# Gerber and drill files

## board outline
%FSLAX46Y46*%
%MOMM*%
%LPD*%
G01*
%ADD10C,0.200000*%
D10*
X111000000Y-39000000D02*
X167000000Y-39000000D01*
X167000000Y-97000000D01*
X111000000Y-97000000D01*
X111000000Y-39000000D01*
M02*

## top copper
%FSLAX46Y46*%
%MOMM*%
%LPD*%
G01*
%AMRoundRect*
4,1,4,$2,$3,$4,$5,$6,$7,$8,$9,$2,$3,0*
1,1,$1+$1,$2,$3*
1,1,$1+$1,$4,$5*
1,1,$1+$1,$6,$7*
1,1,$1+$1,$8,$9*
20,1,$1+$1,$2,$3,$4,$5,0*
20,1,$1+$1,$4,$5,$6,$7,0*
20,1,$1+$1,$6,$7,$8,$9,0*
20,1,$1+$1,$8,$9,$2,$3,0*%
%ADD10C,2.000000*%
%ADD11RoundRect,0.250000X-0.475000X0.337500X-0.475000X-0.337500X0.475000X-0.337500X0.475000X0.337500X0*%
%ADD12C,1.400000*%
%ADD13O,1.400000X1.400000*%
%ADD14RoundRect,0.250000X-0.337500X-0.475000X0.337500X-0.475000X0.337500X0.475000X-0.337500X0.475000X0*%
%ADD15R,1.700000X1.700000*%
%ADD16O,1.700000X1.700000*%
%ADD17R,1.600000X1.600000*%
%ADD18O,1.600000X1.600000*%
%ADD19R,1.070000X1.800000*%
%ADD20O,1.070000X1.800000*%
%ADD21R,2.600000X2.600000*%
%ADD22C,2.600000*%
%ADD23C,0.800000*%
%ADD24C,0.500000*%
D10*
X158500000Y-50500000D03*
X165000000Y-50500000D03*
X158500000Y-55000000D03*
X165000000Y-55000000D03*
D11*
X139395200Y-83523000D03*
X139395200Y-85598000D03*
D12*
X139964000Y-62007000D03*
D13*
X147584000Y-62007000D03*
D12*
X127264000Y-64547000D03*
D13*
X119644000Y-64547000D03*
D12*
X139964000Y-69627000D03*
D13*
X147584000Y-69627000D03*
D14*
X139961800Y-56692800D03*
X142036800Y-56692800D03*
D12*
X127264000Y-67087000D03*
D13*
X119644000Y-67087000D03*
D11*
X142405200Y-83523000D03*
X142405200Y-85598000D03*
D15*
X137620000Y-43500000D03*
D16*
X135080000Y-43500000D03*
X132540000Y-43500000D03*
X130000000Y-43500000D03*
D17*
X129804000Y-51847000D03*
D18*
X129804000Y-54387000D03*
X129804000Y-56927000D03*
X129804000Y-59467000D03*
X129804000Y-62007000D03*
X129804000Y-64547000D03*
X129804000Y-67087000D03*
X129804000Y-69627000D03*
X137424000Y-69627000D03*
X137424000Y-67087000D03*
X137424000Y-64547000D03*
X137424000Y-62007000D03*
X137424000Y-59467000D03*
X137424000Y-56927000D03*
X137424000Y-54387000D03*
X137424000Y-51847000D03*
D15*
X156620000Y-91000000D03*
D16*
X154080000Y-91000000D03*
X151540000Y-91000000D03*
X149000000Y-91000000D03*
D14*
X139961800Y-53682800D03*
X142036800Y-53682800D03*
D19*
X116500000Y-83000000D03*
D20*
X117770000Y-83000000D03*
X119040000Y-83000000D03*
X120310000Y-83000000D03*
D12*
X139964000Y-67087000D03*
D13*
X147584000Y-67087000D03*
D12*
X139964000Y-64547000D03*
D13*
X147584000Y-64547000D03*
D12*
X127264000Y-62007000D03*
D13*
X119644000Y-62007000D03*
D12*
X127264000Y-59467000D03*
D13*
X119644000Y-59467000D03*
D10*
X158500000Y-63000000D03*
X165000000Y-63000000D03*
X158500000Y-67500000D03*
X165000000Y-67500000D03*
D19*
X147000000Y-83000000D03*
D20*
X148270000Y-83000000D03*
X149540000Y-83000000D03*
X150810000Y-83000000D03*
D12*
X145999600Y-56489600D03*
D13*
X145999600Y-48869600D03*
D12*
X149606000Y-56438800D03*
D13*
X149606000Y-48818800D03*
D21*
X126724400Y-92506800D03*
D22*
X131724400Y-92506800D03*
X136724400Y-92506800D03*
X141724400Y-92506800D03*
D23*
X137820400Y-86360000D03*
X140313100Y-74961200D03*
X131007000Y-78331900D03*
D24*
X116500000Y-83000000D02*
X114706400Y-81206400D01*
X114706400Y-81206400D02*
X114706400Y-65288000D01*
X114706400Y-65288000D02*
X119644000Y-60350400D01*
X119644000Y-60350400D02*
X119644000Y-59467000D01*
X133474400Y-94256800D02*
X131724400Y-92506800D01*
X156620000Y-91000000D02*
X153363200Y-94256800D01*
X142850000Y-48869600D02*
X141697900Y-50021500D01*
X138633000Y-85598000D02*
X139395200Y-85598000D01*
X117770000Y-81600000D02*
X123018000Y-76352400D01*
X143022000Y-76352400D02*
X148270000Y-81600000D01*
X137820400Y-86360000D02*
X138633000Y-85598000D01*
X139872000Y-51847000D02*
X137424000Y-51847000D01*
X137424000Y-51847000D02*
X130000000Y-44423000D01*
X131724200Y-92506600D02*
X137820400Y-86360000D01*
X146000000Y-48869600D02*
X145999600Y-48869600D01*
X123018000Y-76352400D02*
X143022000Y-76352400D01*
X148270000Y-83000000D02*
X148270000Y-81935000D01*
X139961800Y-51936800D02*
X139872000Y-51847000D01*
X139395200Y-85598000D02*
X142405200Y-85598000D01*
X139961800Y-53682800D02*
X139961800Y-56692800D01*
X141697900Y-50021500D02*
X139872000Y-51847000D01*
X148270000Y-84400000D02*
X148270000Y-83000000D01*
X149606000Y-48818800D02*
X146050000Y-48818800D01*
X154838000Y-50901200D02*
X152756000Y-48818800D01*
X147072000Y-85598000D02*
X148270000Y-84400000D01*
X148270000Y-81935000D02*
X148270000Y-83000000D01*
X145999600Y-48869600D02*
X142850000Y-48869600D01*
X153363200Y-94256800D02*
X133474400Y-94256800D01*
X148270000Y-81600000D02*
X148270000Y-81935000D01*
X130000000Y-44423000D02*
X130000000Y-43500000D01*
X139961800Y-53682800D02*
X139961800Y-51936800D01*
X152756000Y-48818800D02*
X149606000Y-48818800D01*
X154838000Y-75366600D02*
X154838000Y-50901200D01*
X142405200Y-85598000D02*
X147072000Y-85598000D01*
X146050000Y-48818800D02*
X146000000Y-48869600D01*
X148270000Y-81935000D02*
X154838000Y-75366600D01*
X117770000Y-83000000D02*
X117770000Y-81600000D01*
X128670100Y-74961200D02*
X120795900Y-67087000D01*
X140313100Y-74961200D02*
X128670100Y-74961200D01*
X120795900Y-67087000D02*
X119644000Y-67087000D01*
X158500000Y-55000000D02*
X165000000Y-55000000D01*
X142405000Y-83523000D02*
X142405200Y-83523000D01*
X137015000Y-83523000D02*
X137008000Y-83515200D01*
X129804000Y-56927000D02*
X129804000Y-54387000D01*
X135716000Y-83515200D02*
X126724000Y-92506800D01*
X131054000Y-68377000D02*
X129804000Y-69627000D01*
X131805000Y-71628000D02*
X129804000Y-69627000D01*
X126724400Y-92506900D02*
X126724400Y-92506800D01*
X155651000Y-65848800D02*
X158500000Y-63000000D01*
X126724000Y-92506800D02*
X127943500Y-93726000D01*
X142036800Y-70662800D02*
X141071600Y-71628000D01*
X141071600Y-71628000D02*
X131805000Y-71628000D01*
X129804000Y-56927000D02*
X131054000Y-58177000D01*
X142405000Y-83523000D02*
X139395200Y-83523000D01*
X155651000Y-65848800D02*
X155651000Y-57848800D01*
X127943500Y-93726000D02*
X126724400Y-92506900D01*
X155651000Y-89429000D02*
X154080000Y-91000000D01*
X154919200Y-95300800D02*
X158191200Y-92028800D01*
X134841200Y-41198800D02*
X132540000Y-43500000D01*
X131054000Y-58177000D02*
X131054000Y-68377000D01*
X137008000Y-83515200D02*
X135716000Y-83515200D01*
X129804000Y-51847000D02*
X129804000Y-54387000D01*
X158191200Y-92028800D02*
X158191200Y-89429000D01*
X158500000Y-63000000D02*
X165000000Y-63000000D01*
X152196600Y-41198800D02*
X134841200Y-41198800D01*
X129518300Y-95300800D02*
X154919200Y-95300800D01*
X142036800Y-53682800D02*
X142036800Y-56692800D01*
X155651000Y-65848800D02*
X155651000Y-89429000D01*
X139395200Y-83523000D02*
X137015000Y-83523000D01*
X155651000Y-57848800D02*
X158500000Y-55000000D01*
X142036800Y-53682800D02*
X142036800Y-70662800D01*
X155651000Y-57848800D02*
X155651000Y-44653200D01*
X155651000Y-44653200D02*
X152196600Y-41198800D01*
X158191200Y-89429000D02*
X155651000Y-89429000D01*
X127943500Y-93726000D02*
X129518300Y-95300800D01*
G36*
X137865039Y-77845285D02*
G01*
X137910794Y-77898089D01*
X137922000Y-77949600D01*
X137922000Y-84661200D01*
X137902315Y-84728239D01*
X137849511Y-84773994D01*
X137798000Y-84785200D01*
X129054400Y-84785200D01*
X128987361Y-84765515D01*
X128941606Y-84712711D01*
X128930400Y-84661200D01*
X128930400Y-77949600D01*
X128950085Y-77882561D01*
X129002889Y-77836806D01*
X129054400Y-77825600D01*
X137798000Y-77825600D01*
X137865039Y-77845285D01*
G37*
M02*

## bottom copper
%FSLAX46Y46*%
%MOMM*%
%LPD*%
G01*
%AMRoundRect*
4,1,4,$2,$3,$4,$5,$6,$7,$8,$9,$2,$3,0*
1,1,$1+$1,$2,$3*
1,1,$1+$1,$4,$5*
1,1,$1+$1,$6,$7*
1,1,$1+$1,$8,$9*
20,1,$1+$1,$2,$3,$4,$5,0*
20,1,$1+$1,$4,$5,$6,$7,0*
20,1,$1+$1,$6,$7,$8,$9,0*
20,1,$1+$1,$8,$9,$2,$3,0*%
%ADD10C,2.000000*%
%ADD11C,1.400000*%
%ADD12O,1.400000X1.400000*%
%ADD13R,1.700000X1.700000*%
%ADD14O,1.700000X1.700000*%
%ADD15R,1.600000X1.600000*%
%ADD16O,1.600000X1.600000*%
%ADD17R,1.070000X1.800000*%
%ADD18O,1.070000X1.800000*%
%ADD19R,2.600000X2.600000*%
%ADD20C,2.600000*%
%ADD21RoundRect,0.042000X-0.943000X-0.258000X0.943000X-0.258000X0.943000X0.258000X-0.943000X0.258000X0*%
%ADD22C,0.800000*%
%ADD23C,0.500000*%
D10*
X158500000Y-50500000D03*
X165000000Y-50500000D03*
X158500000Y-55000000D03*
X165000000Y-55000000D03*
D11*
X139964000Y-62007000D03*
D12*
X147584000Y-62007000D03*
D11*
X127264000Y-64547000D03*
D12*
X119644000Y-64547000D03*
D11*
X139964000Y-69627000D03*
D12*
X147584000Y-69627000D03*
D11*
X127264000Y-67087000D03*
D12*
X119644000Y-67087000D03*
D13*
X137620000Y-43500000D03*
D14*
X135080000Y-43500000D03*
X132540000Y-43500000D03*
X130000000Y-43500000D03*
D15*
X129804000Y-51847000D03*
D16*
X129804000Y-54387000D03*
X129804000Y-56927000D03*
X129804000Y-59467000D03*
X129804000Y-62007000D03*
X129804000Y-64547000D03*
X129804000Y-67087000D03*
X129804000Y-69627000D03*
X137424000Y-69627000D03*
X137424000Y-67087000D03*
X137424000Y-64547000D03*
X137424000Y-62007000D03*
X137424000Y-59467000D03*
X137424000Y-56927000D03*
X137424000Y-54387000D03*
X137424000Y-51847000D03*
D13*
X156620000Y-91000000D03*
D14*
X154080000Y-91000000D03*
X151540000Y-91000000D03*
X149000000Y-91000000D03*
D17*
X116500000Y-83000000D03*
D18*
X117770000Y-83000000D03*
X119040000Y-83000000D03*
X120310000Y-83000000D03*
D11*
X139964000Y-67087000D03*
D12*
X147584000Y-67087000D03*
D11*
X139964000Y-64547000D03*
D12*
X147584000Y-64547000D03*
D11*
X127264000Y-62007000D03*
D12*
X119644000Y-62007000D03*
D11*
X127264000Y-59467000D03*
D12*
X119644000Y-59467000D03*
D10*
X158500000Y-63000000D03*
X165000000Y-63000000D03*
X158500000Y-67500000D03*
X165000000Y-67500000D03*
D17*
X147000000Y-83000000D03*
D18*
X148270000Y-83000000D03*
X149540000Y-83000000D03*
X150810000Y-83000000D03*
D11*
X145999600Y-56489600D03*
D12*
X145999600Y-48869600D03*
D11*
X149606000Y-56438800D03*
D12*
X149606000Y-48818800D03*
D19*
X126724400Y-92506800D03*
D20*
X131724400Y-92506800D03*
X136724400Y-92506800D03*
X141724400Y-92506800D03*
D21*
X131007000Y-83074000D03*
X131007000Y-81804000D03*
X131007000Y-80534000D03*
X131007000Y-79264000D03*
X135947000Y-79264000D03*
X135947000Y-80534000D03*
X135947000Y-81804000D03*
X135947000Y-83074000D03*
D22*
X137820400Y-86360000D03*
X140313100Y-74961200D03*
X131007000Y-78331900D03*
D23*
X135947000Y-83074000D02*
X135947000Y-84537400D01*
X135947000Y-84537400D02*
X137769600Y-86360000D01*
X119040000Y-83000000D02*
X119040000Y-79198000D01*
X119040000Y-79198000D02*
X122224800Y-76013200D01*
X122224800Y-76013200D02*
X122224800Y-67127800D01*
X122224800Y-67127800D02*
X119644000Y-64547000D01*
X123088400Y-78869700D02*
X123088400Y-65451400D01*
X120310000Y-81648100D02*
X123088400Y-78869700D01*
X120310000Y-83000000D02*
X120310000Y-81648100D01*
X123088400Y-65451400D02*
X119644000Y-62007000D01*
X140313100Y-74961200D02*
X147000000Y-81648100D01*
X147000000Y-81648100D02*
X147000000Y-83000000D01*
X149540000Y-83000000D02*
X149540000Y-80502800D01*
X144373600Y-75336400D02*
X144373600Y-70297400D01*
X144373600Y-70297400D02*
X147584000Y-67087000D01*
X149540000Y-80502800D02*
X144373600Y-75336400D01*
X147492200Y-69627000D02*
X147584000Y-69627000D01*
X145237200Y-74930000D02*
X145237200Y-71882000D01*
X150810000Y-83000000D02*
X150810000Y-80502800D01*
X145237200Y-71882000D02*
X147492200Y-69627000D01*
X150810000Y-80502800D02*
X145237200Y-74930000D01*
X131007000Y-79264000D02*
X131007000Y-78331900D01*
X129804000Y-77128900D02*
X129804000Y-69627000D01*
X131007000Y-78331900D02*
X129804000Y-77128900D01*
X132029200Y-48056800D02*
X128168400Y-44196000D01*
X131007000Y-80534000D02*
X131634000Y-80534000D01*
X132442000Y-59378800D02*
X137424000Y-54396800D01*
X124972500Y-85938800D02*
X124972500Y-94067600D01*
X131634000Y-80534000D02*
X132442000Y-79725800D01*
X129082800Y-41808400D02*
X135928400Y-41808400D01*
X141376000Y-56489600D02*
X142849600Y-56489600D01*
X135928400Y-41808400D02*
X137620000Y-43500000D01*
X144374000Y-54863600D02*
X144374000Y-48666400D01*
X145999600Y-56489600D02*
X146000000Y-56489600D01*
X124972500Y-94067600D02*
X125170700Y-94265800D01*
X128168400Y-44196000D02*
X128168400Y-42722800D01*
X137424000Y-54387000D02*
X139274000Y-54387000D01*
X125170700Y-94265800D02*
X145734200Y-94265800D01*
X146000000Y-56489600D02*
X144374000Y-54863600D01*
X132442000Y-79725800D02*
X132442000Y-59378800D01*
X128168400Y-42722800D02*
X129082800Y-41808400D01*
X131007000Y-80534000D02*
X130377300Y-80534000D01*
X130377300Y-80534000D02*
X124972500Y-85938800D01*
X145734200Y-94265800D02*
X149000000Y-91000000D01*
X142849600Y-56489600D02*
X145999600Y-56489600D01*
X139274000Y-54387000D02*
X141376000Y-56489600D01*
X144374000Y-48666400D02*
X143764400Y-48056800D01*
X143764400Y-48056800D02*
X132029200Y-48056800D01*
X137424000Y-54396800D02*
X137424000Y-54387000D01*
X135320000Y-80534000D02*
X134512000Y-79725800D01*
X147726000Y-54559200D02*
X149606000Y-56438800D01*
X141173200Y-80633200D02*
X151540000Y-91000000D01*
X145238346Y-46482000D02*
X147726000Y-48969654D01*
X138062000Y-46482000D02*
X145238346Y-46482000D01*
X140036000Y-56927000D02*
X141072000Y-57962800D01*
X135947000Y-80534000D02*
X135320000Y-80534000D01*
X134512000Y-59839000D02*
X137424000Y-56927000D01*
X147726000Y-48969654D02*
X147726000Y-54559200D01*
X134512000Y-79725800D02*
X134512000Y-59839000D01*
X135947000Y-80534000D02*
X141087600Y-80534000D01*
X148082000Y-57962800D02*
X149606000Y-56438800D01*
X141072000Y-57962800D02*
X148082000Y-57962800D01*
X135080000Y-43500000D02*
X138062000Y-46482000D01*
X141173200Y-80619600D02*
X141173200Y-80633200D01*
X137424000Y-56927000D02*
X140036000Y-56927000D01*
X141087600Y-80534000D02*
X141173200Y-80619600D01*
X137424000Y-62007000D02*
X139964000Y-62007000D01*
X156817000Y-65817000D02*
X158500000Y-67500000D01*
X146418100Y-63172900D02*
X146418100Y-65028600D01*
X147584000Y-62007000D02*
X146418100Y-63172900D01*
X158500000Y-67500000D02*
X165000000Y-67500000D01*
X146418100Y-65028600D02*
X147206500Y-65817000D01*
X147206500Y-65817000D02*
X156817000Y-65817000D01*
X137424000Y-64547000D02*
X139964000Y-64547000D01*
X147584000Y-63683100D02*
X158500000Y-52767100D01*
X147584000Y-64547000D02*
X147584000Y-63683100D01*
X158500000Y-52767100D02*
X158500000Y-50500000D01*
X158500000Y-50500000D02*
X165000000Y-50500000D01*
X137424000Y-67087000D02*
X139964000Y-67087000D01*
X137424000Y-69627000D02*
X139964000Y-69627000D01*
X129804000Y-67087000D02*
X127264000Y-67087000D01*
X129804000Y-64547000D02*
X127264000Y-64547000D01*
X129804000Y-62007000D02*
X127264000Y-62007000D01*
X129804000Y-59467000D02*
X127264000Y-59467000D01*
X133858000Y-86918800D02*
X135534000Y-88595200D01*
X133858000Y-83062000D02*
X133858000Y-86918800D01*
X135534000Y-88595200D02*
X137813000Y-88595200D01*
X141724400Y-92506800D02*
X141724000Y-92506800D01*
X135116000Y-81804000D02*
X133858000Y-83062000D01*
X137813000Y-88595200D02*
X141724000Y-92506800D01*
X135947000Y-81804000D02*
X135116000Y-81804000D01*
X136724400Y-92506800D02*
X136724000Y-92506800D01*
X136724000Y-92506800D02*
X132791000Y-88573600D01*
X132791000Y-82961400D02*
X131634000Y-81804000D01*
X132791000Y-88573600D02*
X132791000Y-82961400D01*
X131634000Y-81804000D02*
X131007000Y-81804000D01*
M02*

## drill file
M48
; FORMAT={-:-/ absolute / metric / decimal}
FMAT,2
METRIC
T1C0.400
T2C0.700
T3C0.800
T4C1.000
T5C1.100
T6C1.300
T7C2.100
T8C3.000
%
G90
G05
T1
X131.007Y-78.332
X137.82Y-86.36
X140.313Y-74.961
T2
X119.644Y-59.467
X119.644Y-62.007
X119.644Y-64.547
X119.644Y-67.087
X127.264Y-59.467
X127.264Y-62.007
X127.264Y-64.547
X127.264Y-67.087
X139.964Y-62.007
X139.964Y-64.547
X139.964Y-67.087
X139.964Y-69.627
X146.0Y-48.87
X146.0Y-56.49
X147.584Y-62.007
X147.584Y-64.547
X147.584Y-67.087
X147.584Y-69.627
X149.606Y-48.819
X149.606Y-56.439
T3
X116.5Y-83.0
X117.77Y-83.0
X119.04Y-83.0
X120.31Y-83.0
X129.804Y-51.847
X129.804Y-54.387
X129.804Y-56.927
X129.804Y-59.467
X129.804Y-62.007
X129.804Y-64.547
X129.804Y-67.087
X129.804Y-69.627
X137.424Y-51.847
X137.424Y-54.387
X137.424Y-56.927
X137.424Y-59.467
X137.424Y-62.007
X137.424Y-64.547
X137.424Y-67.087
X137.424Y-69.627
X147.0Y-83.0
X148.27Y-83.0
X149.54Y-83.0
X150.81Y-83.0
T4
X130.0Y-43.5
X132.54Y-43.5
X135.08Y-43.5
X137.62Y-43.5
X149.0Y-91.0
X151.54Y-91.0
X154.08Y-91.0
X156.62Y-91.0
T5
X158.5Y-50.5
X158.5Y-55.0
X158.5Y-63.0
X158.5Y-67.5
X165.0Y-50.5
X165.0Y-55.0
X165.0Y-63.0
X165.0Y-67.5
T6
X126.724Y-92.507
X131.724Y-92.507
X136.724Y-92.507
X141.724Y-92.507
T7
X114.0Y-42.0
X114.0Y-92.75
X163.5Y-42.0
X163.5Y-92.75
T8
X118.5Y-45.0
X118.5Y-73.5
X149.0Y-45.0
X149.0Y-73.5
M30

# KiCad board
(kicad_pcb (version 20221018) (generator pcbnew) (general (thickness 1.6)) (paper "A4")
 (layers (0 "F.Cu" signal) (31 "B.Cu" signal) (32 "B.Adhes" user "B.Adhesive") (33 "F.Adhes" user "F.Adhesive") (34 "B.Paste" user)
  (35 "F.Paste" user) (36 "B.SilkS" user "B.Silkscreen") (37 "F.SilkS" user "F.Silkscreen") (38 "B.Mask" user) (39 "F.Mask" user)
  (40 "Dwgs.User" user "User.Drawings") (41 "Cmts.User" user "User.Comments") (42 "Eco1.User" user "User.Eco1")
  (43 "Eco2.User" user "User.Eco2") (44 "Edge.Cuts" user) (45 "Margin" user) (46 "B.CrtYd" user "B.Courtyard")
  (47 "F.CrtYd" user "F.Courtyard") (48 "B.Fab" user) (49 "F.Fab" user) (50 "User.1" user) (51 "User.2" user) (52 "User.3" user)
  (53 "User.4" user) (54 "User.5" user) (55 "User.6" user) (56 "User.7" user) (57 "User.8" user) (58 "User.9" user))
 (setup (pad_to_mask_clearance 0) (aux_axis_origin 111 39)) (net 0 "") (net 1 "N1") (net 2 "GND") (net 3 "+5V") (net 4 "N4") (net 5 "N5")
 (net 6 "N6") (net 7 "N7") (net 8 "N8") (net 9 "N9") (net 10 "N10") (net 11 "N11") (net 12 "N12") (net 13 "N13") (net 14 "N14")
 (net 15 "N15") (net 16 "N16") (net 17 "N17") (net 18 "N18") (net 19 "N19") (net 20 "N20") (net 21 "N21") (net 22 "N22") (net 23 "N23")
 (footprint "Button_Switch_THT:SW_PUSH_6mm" (layer "F.Cu") (at 158.5 50.5)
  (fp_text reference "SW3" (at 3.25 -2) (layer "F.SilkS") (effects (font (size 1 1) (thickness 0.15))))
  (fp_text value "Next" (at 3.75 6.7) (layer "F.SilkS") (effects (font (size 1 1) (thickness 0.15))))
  (pad "1" thru_hole circle (at 0 0 90) (size 2 2) (drill 1.1) (layers "*.Cu" "*.Mask") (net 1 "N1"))
  (pad "1" thru_hole circle (at 6.5 0 90) (size 2 2) (drill 1.1) (layers "*.Cu" "*.Mask") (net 1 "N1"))
  (pad "2" thru_hole circle (at 0 4.5 90) (size 2 2) (drill 1.1) (layers "*.Cu" "*.Mask") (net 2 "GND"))
  (pad "2" thru_hole circle (at 6.5 4.5 90) (size 2 2) (drill 1.1) (layers "*.Cu" "*.Mask") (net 2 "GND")))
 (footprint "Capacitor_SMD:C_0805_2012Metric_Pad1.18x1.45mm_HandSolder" (layer "F.Cu") (at 139.3952 84.5605 -90)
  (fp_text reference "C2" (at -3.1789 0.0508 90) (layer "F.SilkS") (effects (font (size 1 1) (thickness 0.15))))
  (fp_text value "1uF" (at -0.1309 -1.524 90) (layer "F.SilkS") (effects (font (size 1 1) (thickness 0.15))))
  (pad "1" smd roundrect (at -1.0375 0 270) (size 1.175 1.45) (layers "F.Cu" "F.Paste" "F.Mask") (roundrect_rratio 0.2127659574)
   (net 2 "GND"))
  (pad "2" smd roundrect (at 1.0375 0 270) (size 1.175 1.45) (layers "F.Cu" "F.Paste" "F.Mask") (roundrect_rratio 0.2127659574)
   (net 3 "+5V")))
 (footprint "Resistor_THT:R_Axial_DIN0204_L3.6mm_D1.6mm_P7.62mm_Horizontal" (layer "F.Cu") (at 139.964 62.007)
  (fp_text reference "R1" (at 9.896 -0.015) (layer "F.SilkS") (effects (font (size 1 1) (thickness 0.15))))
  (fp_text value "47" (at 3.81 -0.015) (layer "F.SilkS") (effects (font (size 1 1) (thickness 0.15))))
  (pad "1" thru_hole circle (at 0 0) (size 1.4 1.4) (drill 0.7) (layers "*.Cu" "*.Mask") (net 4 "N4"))
  (pad "2" thru_hole oval (at 7.62 0) (size 1.4 1.4) (drill 0.7) (layers "*.Cu" "*.Mask") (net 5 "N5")))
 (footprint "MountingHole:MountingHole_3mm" (layer "F.Cu") (at 149 73.5)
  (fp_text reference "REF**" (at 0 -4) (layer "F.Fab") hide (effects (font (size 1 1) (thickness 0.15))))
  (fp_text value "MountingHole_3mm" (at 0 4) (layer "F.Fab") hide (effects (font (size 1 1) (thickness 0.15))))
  (pad "" np_thru_hole circle (at 0 0) (size 3 3) (drill 3) (layers "*.Cu" "*.Mask")))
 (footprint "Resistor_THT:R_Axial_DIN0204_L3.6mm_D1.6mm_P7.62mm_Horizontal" (layer "F.Cu") (at 127.264 64.547 180)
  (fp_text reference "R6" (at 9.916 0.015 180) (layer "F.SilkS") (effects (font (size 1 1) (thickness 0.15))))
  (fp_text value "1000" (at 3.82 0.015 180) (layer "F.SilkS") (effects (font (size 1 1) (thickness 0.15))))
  (pad "1" thru_hole circle (at 0 0 180) (size 1.4 1.4) (drill 0.7) (layers "*.Cu" "*.Mask") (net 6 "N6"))
  (pad "2" thru_hole oval (at 7.62 0 180) (size 1.4 1.4) (drill 0.7) (layers "*.Cu" "*.Mask") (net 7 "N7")))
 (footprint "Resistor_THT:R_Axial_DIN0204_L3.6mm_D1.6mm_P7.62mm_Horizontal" (layer "F.Cu") (at 139.964 69.627)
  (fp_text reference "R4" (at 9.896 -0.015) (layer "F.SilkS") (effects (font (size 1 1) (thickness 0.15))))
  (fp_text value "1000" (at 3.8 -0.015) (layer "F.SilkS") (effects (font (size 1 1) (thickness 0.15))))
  (pad "1" thru_hole circle (at 0 0) (size 1.4 1.4) (drill 0.7) (layers "*.Cu" "*.Mask") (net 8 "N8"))
  (pad "2" thru_hole oval (at 7.62 0) (size 1.4 1.4) (drill 0.7) (layers "*.Cu" "*.Mask") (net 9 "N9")))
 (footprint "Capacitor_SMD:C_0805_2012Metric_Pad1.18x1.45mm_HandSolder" (layer "F.Cu") (at 140.9993 56.6928)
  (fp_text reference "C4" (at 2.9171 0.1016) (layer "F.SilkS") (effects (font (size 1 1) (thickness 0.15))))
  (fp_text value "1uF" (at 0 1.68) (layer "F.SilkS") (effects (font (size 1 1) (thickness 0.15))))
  (pad "1" smd roundrect (at -1.0375 0) (size 1.175 1.45) (layers "F.Cu" "F.Paste" "F.Mask") (roundrect_rratio 0.2127659574) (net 3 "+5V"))
  (pad "2" smd roundrect (at 1.0375 0) (size 1.175 1.45) (layers "F.Cu" "F.Paste" "F.Mask") (roundrect_rratio 0.2127659574) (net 2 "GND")))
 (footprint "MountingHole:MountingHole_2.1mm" (layer "F.Cu") (at 114 92.75)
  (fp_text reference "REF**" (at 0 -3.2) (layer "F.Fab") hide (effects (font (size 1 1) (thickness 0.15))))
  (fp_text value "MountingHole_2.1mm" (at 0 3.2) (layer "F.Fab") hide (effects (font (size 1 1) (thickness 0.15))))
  (pad "" np_thru_hole circle (at 0 0) (size 2.1 2.1) (drill 2.1) (layers "F&B.Cu" "*.Mask")))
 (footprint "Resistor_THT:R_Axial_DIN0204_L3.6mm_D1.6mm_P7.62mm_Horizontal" (layer "F.Cu") (at 127.264 67.087 180)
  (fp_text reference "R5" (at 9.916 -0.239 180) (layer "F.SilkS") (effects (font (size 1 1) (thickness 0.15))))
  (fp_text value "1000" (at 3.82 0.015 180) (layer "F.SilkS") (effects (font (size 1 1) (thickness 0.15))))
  (pad "1" thru_hole circle (at 0 0 180) (size 1.4 1.4) (drill 0.7) (layers "*.Cu" "*.Mask") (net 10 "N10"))
  (pad "2" thru_hole oval (at 7.62 0 180) (size 1.4 1.4) (drill 0.7) (layers "*.Cu" "*.Mask") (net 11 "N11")))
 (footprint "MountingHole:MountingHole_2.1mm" (layer "F.Cu") (at 114 42)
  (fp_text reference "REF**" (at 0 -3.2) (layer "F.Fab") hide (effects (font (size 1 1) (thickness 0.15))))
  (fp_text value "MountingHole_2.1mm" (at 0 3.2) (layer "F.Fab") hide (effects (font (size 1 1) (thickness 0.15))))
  (pad "" np_thru_hole circle (at 0 0) (size 2.1 2.1) (drill 2.1) (layers "*.Cu" "*.Mask")))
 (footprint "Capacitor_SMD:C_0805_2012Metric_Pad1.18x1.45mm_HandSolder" (layer "F.Cu") (at 142.4052 84.5605 -90)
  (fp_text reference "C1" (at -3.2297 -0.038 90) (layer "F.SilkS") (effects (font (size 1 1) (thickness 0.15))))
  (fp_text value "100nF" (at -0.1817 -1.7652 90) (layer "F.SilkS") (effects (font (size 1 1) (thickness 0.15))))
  (pad "1" smd roundrect (at -1.0375 0 270) (size 1.175 1.45) (layers "F.Cu" "F.Paste" "F.Mask") (roundrect_rratio 0.2127659574)
   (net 2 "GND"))
  (pad "2" smd roundrect (at 1.0375 0 270) (size 1.175 1.45) (layers "F.Cu" "F.Paste" "F.Mask") (roundrect_rratio 0.2127659574)
   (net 3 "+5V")))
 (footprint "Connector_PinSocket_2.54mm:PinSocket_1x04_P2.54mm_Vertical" (layer "F.Cu") (at 137.62 43.5 -90)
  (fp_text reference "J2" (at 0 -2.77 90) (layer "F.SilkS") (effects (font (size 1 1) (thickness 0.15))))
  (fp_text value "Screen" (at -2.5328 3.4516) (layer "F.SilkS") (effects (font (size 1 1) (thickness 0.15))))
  (pad "1" thru_hole rect (at 0 0 270) (size 1.7 1.7) (drill 1) (layers "*.Cu" "*.Mask") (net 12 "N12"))
  (pad "2" thru_hole oval (at 0 2.54 270) (size 1.7 1.7) (drill 1) (layers "*.Cu" "*.Mask") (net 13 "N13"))
  (pad "3" thru_hole oval (at 0 5.08 270) (size 1.7 1.7) (drill 1) (layers "*.Cu" "*.Mask") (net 2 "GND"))
  (pad "4" thru_hole oval (at 0 7.62 270) (size 1.7 1.7) (drill 1) (layers "*.Cu" "*.Mask") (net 3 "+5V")))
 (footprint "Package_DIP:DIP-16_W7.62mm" (layer "F.Cu") (at 129.804 51.847)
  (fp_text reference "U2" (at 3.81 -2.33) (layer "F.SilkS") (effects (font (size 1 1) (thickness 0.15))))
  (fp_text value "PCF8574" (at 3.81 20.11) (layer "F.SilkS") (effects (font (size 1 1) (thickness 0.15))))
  (pad "1" thru_hole rect (at 0 0) (size 1.6 1.6) (drill 0.8) (layers "*.Cu" "*.Mask") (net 2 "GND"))
  (pad "2" thru_hole oval (at 0 2.54) (size 1.6 1.6) (drill 0.8) (layers "*.Cu" "*.Mask") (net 2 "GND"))
  (pad "3" thru_hole oval (at 0 5.08) (size 1.6 1.6) (drill 0.8) (layers "*.Cu" "*.Mask") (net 2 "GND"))
  (pad "4" thru_hole oval (at 0 7.62) (size 1.6 1.6) (drill 0.8) (layers "*.Cu" "*.Mask") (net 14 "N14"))
  (pad "5" thru_hole oval (at 0 10.16) (size 1.6 1.6) (drill 0.8) (layers "*.Cu" "*.Mask") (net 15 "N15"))
  (pad "6" thru_hole oval (at 0 12.7) (size 1.6 1.6) (drill 0.8) (layers "*.Cu" "*.Mask") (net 6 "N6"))
  (pad "7" thru_hole oval (at 0 15.24) (size 1.6 1.6) (drill 0.8) (layers "*.Cu" "*.Mask") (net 10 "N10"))
  (pad "8" thru_hole oval (at 0 17.78) (size 1.6 1.6) (drill 0.8) (layers "*.Cu" "*.Mask") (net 2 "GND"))
  (pad "9" thru_hole oval (at 7.62 17.78) (size 1.6 1.6) (drill 0.8) (layers "*.Cu" "*.Mask") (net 8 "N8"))
  (pad "10" thru_hole oval (at 7.62 15.24) (size 1.6 1.6) (drill 0.8) (layers "*.Cu" "*.Mask") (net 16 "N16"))
  (pad "11" thru_hole oval (at 7.62 12.7) (size 1.6 1.6) (drill 0.8) (layers "*.Cu" "*.Mask") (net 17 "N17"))
  (pad "12" thru_hole oval (at 7.62 10.16) (size 1.6 1.6) (drill 0.8) (layers "*.Cu" "*.Mask") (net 4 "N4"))
  (pad "13" thru_hole oval (at 7.62 7.62) (size 1.6 1.6) (drill 0.8) (layers "*.Cu" "*.Mask") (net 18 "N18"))
  (pad "14" thru_hole oval (at 7.62 5.08) (size 1.6 1.6) (drill 0.8) (layers "*.Cu" "*.Mask") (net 13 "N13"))
  (pad "15" thru_hole oval (at 7.62 2.54) (size 1.6 1.6) (drill 0.8) (layers "*.Cu" "*.Mask") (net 12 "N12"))
  (pad "16" thru_hole oval (at 7.62 0) (size 1.6 1.6) (drill 0.8) (layers "*.Cu" "*.Mask") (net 3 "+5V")))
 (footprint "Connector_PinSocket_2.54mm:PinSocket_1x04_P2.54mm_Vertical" (layer "F.Cu") (at 156.62 91 -90)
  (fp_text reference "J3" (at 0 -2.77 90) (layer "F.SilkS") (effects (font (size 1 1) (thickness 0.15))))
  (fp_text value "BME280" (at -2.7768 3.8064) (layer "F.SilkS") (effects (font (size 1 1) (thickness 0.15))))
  (pad "1" thru_hole rect (at 0 0 270) (size 1.7 1.7) (drill 1) (layers "*.Cu" "*.Mask") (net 3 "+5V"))
  (pad "2" thru_hole oval (at 0 2.54 270) (size 1.7 1.7) (drill 1) (layers "*.Cu" "*.Mask") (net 2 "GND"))
  (pad "3" thru_hole oval (at 0 5.08 270) (size 1.7 1.7) (drill 1) (layers "*.Cu" "*.Mask") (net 13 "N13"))
  (pad "4" thru_hole oval (at 0 7.62 270) (size 1.7 1.7) (drill 1) (layers "*.Cu" "*.Mask") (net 12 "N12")))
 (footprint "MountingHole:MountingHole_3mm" (layer "F.Cu") (at 149 45)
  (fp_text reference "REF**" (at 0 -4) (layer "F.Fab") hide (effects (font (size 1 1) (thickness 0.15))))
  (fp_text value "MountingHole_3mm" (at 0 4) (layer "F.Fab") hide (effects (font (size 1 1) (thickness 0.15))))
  (pad "" np_thru_hole circle (at 0 0) (size 3 3) (drill 3) (layers "*.Cu" "*.Mask")))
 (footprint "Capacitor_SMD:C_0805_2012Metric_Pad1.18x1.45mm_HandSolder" (layer "F.Cu") (at 140.9993 53.6828)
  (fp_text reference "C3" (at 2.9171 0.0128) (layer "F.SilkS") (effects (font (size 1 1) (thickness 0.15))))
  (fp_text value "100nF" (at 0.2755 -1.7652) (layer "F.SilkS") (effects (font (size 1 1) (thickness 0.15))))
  (pad "1" smd roundrect (at -1.0375 0) (size 1.175 1.45) (layers "F.Cu" "F.Paste" "F.Mask") (roundrect_rratio 0.2127659574) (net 3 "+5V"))
  (pad "2" smd roundrect (at 1.0375 0) (size 1.175 1.45) (layers "F.Cu" "F.Paste" "F.Mask") (roundrect_rratio 0.2127659574) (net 2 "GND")))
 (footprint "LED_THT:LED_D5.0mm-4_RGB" (layer "F.Cu") (at 116.5 83)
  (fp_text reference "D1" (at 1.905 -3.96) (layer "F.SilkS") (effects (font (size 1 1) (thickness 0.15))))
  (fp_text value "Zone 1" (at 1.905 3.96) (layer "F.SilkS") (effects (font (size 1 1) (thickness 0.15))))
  (pad "1" thru_hole rect (at 0 0) (size 1.07 1.8) (drill 0.8) (layers "*.Cu" "*.Mask") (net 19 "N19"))
  (pad "2" thru_hole oval (at 1.27 0) (size 1.07 1.8) (drill 0.8) (layers "*.Cu" "*.Mask") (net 3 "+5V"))
  (pad "3" thru_hole oval (at 2.54 0) (size 1.07 1.8) (drill 0.8) (layers "*.Cu" "*.Mask") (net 7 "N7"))
  (pad "4" thru_hole oval (at 3.81 0) (size 1.07 1.8) (drill 0.8) (layers "*.Cu" "*.Mask") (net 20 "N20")))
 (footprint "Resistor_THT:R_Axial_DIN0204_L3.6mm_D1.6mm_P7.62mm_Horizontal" (layer "F.Cu") (at 139.964 67.087)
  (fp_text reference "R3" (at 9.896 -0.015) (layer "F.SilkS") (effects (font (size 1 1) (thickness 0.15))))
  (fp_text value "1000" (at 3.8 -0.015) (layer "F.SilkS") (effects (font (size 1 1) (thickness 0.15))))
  (pad "1" thru_hole circle (at 0 0) (size 1.4 1.4) (drill 0.7) (layers "*.Cu" "*.Mask") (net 16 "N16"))
  (pad "2" thru_hole oval (at 7.62 0) (size 1.4 1.4) (drill 0.7) (layers "*.Cu" "*.Mask") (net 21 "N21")))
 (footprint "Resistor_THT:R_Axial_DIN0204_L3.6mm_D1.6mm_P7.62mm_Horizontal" (layer "F.Cu") (at 139.964 64.547)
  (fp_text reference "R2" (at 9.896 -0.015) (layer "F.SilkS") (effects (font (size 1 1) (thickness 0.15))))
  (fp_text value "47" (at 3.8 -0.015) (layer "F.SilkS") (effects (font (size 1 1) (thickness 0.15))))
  (pad "1" thru_hole circle (at 0 0) (size 1.4 1.4) (drill 0.7) (layers "*.Cu" "*.Mask") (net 17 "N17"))
  (pad "2" thru_hole oval (at 7.62 0) (size 1.4 1.4) (drill 0.7) (layers "*.Cu" "*.Mask") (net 1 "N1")))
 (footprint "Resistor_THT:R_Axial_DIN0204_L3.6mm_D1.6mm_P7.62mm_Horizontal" (layer "F.Cu") (at 127.264 62.007 180)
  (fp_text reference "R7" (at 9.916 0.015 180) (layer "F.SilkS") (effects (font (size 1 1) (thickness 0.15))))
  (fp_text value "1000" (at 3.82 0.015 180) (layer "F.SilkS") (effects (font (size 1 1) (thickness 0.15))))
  (pad "1" thru_hole circle (at 0 0 180) (size 1.4 1.4) (drill 0.7) (layers "*.Cu" "*.Mask") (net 15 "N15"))
  (pad "2" thru_hole oval (at 7.62 0 180) (size 1.4 1.4) (drill 0.7) (layers "*.Cu" "*.Mask") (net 20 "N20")))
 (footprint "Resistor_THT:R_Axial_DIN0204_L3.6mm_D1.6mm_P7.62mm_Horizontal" (layer "F.Cu") (at 127.264 59.467 180)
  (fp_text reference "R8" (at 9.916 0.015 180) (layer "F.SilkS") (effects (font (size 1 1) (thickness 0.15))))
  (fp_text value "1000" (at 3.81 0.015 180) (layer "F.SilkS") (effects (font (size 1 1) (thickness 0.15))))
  (pad "1" thru_hole circle (at 0 0 180) (size 1.4 1.4) (drill 0.7) (layers "*.Cu" "*.Mask") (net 14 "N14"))
  (pad "2" thru_hole oval (at 7.62 0 180) (size 1.4 1.4) (drill 0.7) (layers "*.Cu" "*.Mask") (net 19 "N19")))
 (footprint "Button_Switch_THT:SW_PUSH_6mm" (layer "F.Cu") (at 158.5 63)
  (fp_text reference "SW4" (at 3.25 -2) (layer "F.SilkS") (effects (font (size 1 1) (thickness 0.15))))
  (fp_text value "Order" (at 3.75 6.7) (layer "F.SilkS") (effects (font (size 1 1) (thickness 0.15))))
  (pad "1" thru_hole circle (at 0 0 90) (size 2 2) (drill 1.1) (layers "*.Cu" "*.Mask") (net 2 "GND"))
  (pad "1" thru_hole circle (at 6.5 0 90) (size 2 2) (drill 1.1) (layers "*.Cu" "*.Mask") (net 2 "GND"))
  (pad "2" thru_hole circle (at 0 4.5 90) (size 2 2) (drill 1.1) (layers "*.Cu" "*.Mask") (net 5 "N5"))
  (pad "2" thru_hole circle (at 6.5 4.5 90) (size 2 2) (drill 1.1) (layers "*.Cu" "*.Mask") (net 5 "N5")))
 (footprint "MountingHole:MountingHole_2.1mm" (layer "F.Cu") (at 163.5 92.75)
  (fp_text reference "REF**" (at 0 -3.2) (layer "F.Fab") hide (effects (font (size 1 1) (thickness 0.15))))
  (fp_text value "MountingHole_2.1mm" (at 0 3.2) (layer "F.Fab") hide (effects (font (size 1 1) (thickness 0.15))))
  (pad "" np_thru_hole circle (at 0 0) (size 2.1 2.1) (drill 2.1) (layers "F&B.Cu" "*.Mask")))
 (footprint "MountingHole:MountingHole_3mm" (layer "F.Cu") (at 118.5 73.5)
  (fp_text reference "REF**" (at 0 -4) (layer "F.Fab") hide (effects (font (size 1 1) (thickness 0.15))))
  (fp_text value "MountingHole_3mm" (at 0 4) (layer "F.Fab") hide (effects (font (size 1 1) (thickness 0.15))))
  (pad "" np_thru_hole circle (at 0 0) (size 3 3) (drill 3) (layers "*.Cu" "*.Mask")))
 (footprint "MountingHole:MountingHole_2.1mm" (layer "F.Cu") (at 163.5 42)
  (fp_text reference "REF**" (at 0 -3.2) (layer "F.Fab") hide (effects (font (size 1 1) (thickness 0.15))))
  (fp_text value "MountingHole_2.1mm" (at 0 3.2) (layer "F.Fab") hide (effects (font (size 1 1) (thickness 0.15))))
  (pad "" np_thru_hole circle (at 0 0) (size 2.1 2.1) (drill 2.1) (layers "F&B.Cu" "*.Mask")))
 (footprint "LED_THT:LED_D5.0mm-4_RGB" (layer "F.Cu") (at 147 83)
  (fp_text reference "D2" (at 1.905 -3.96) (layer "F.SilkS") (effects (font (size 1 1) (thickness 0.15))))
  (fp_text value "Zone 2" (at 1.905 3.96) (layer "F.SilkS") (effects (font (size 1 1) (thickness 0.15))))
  (pad "1" thru_hole rect (at 0 0) (size 1.07 1.8) (drill 0.8) (layers "*.Cu" "*.Mask") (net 11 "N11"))
  (pad "2" thru_hole oval (at 1.27 0) (size 1.07 1.8) (drill 0.8) (layers "*.Cu" "*.Mask") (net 3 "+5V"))
  (pad "3" thru_hole oval (at 2.54 0) (size 1.07 1.8) (drill 0.8) (layers "*.Cu" "*.Mask") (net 21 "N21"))
  (pad "4" thru_hole oval (at 3.81 0) (size 1.07 1.8) (drill 0.8) (layers "*.Cu" "*.Mask") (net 9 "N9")))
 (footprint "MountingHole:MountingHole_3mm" (layer "F.Cu") (at 118.5 45)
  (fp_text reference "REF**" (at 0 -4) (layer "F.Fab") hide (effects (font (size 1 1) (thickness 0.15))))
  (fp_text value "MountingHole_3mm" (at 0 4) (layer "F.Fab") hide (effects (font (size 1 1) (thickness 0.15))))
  (pad "" np_thru_hole circle (at 0 0) (size 3 3) (drill 3) (layers "*.Cu" "*.Mask")))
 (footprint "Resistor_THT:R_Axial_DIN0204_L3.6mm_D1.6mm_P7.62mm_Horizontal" (layer "B.Cu") (at 145.9996 56.4896 90)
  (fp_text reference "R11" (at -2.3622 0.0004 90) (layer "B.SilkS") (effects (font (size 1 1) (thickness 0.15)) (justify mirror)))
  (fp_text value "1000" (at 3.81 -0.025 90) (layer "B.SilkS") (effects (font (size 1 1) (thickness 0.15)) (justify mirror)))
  (pad "1" thru_hole circle (at 0 0 90) (size 1.4 1.4) (drill 0.7) (layers "*.Cu" "*.Mask") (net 12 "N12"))
  (pad "2" thru_hole oval (at 7.62 0 90) (size 1.4 1.4) (drill 0.7) (layers "*.Cu" "*.Mask") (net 3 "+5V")))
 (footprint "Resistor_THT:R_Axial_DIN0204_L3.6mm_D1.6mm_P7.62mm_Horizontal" (layer "B.Cu") (at 149.606 56.4388 90)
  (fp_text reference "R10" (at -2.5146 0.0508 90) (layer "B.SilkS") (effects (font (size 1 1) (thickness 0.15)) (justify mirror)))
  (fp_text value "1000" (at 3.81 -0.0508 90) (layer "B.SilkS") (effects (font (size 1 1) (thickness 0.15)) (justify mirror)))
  (pad "1" thru_hole circle (at 0 0 90) (size 1.4 1.4) (drill 0.7) (layers "*.Cu" "*.Mask") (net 13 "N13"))
  (pad "2" thru_hole oval (at 7.62 0 90) (size 1.4 1.4) (drill 0.7) (layers "*.Cu" "*.Mask") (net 3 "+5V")))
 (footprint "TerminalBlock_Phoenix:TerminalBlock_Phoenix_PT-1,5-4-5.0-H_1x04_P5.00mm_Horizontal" (layer "B.Cu") (at 126.7244 92.5068)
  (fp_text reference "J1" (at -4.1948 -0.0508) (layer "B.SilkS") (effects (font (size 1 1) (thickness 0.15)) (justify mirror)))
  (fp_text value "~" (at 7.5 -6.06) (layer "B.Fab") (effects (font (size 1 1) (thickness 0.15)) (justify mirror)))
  (pad "1" thru_hole rect (at 0 0) (size 2.6 2.6) (drill 1.3) (layers "*.Cu" "*.Mask") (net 2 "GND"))
  (pad "2" thru_hole circle (at 5 0) (size 2.6 2.6) (drill 1.3) (layers "*.Cu" "*.Mask") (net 3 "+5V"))
  (pad "3" thru_hole circle (at 10 0) (size 2.6 2.6) (drill 1.3) (layers "*.Cu" "*.Mask") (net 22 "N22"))
  (pad "4" thru_hole circle (at 15 0) (size 2.6 2.6) (drill 1.3) (layers "*.Cu" "*.Mask") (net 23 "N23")))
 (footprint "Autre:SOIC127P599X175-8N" (layer "B.Cu") (at 133.477 81.169)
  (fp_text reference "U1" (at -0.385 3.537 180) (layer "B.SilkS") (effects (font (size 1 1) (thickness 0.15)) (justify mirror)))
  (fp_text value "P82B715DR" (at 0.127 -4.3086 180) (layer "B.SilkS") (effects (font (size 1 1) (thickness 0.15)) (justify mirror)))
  (pad "1" smd roundrect (at -2.47 1.905) (size 1.97 0.6) (layers "B.Cu" "B.Paste" "B.Mask") (roundrect_rratio 0.07))
  (pad "2" smd roundrect (at -2.47 0.635) (size 1.97 0.6) (layers "B.Cu" "B.Paste" "B.Mask") (roundrect_rratio 0.07) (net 22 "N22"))
  (pad "3" smd roundrect (at -2.47 -0.635) (size 1.97 0.6) (layers "B.Cu" "B.Paste" "B.Mask") (roundrect_rratio 0.07) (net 12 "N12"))
  (pad "4" smd roundrect (at -2.47 -1.905) (size 1.97 0.6) (layers "B.Cu" "B.Paste" "B.Mask") (roundrect_rratio 0.07) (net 2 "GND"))
  (pad "5" smd roundrect (at 2.47 -1.905) (size 1.97 0.6) (layers "B.Cu" "B.Paste" "B.Mask") (roundrect_rratio 0.07))
  (pad "6" smd roundrect (at 2.47 -0.635) (size 1.97 0.6) (layers "B.Cu" "B.Paste" "B.Mask") (roundrect_rratio 0.07) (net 13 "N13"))
  (pad "7" smd roundrect (at 2.47 0.635) (size 1.97 0.6) (layers "B.Cu" "B.Paste" "B.Mask") (roundrect_rratio 0.07) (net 23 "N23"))
  (pad "8" smd roundrect (at 2.47 1.905) (size 1.97 0.6) (layers "B.Cu" "B.Paste" "B.Mask") (roundrect_rratio 0.07) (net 3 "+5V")))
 (gr_rect (start 111 39) (end 167 97) (stroke (width 0.2) (type default)) (fill none) (layer "Edge.Cuts"))
 (segment (start 116.5 83) (end 114.7064 81.2064) (width 0.5) (layer "F.Cu") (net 19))
 (segment (start 114.7064 81.2064) (end 114.7064 65.288) (width 0.5) (layer "F.Cu") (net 19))
 (segment (start 114.7064 65.288) (end 119.644 60.3504) (width 0.5) (layer "F.Cu") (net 19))
 (segment (start 119.644 60.3504) (end 119.644 59.467) (width 0.5) (layer "F.Cu") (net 19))
 (segment (start 133.4744 94.2568) (end 131.7244 92.5068) (width 0.5) (layer "F.Cu") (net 3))
 (segment (start 156.62 91) (end 153.3632 94.2568) (width 0.5) (layer "F.Cu") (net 3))
 (segment (start 142.85 48.8696) (end 141.6979 50.0215) (width 0.5) (layer "F.Cu") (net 3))
 (segment (start 138.633 85.598) (end 139.3952 85.598) (width 0.5) (layer "F.Cu") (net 3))
 (segment (start 117.77 81.6) (end 123.018 76.3524) (width 0.5) (layer "F.Cu") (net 3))
 (segment (start 143.022 76.3524) (end 148.27 81.6) (width 0.5) (layer "F.Cu") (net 3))
 (segment (start 137.8204 86.36) (end 138.633 85.598) (width 0.5) (layer "F.Cu") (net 3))
 (segment (start 139.872 51.847) (end 137.424 51.847) (width 0.5) (layer "F.Cu") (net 3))
 (segment (start 137.424 51.847) (end 130 44.423) (width 0.5) (layer "F.Cu") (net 3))
 (segment (start 131.7242 92.5066) (end 137.8204 86.36) (width 0.5) (layer "F.Cu") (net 3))
 (segment (start 146 48.8696) (end 145.9996 48.8696) (width 0.5) (layer "F.Cu") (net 3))
 (segment (start 123.018 76.3524) (end 143.022 76.3524) (width 0.5) (layer "F.Cu") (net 3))
 (segment (start 148.27 83) (end 148.27 81.935) (width 0.5) (layer "F.Cu") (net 3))
 (segment (start 139.9618 51.9368) (end 139.872 51.847) (width 0.5) (layer "F.Cu") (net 3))
 (segment (start 139.3952 85.598) (end 142.4052 85.598) (width 0.5) (layer "F.Cu") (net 3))
 (segment (start 139.9618 53.6828) (end 139.9618 56.6928) (width 0.5) (layer "F.Cu") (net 3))
 (segment (start 141.6979 50.0215) (end 139.872 51.847) (width 0.5) (layer "F.Cu") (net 3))
 (segment (start 148.27 84.4) (end 148.27 83) (width 0.5) (layer "F.Cu") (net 3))
 (segment (start 149.606 48.8188) (end 146.05 48.8188) (width 0.5) (layer "F.Cu") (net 3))
 (segment (start 154.838 50.9012) (end 152.756 48.8188) (width 0.5) (layer "F.Cu") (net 3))
 (segment (start 147.072 85.598) (end 148.27 84.4) (width 0.5) (layer "F.Cu") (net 3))
 (segment (start 148.27 81.935) (end 148.27 83) (width 0.5) (layer "F.Cu") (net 3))
 (segment (start 145.9996 48.8696) (end 142.85 48.8696) (width 0.5) (layer "F.Cu") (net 3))
 (segment (start 153.3632 94.2568) (end 133.4744 94.2568) (width 0.5) (layer "F.Cu") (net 3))
 (segment (start 148.27 81.6) (end 148.27 81.935) (width 0.5) (layer "F.Cu") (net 3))
 (segment (start 130 44.423) (end 130 43.5) (width 0.5) (layer "F.Cu") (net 3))
 (segment (start 139.9618 53.6828) (end 139.9618 51.9368) (width 0.5) (layer "F.Cu") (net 3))
 (segment (start 152.756 48.8188) (end 149.606 48.8188) (width 0.5) (layer "F.Cu") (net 3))
 (segment (start 154.838 75.3666) (end 154.838 50.9012) (width 0.5) (layer "F.Cu") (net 3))
 (segment (start 142.4052 85.598) (end 147.072 85.598) (width 0.5) (layer "F.Cu") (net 3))
 (segment (start 146.05 48.8188) (end 146 48.8696) (width 0.5) (layer "F.Cu") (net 3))
 (segment (start 148.27 81.935) (end 154.838 75.3666) (width 0.5) (layer "F.Cu") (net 3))
 (segment (start 117.77 83) (end 117.77 81.6) (width 0.5) (layer "F.Cu") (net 3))
 (via (at 137.8204 86.36) (size 0.8) (drill 0.4) (layers "F.Cu" "B.Cu") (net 3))
 (segment (start 135.947 83.074) (end 135.947 84.5374) (width 0.5) (layer "B.Cu") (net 3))
 (segment (start 135.947 84.5374) (end 137.7696 86.36) (width 0.5) (layer "B.Cu") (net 3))
 (segment (start 119.04 83) (end 119.04 79.198) (width 0.5) (layer "B.Cu") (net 7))
 (segment (start 119.04 79.198) (end 122.2248 76.0132) (width 0.5) (layer "B.Cu") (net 7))
 (segment (start 122.2248 76.0132) (end 122.2248 67.1278) (width 0.5) (layer "B.Cu") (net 7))
 (segment (start 122.2248 67.1278) (end 119.644 64.547) (width 0.5) (layer "B.Cu") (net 7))
 (segment (start 123.0884 78.8697) (end 123.0884 65.4514) (width 0.5) (layer "B.Cu") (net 20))
 (segment (start 120.31 81.6481) (end 123.0884 78.8697) (width 0.5) (layer "B.Cu") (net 20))
 (segment (start 120.31 83) (end 120.31 81.6481) (width 0.5) (layer "B.Cu") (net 20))
 (segment (start 123.0884 65.4514) (end 119.644 62.007) (width 0.5) (layer "B.Cu") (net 20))
 (segment (start 128.6701 74.9612) (end 120.7959 67.087) (width 0.5) (layer "F.Cu") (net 11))
 (segment (start 140.3131 74.9612) (end 128.6701 74.9612) (width 0.5) (layer "F.Cu") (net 11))
 (segment (start 120.7959 67.087) (end 119.644 67.087) (width 0.5) (layer "F.Cu") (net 11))
 (via (at 140.3131 74.9612) (size 0.8) (drill 0.4) (layers "F.Cu" "B.Cu") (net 11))
 (segment (start 140.3131 74.9612) (end 147 81.6481) (width 0.5) (layer "B.Cu") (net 11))
 (segment (start 147 81.6481) (end 147 83) (width 0.5) (layer "B.Cu") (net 11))
 (segment (start 149.54 83) (end 149.54 80.5028) (width 0.5) (layer "B.Cu") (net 21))
 (segment (start 144.3736 75.3364) (end 144.3736 70.2974) (width 0.5) (layer "B.Cu") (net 21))
 (segment (start 144.3736 70.2974) (end 147.584 67.087) (width 0.5) (layer "B.Cu") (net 21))
 (segment (start 149.54 80.5028) (end 144.3736 75.3364) (width 0.5) (layer "B.Cu") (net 21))
 (segment (start 147.4922 69.627) (end 147.584 69.627) (width 0.5) (layer "B.Cu") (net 9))
 (segment (start 145.2372 74.93) (end 145.2372 71.882) (width 0.5) (layer "B.Cu") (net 9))
 (segment (start 150.81 83) (end 150.81 80.5028) (width 0.5) (layer "B.Cu") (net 9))
 (segment (start 145.2372 71.882) (end 147.4922 69.627) (width 0.5) (layer "B.Cu") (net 9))
 (segment (start 150.81 80.5028) (end 145.2372 74.93) (width 0.5) (layer "B.Cu") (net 9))
 (segment (start 158.5 55) (end 165 55) (width 0.5) (layer "F.Cu") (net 2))
 (segment (start 142.405 83.523) (end 142.4052 83.523) (width 0.5) (layer "F.Cu") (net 2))
 (segment (start 137.015 83.523) (end 137.008 83.5152) (width 0.5) (layer "F.Cu") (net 2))
 (segment (start 129.804 56.927) (end 129.804 54.387) (width 0.5) (layer "F.Cu") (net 2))
 (segment (start 135.716 83.5152) (end 126.724 92.5068) (width 0.5) (layer "F.Cu") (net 2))
 (segment (start 131.054 68.377) (end 129.804 69.627) (width 0.5) (layer "F.Cu") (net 2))
 (segment (start 131.805 71.628) (end 129.804 69.627) (width 0.5) (layer "F.Cu") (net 2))
 (segment (start 126.7244 92.5069) (end 126.7244 92.5068) (width 0.5) (layer "F.Cu") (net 2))
 (segment (start 155.651 65.8488) (end 158.5 63) (width 0.5) (layer "F.Cu") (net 2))
 (segment (start 126.724 92.5068) (end 127.9435 93.726) (width 0.5) (layer "F.Cu") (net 2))
 (segment (start 142.0368 70.6628) (end 141.0716 71.628) (width 0.5) (layer "F.Cu") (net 2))
 (segment (start 141.0716 71.628) (end 131.805 71.628) (width 0.5) (layer "F.Cu") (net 2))
 (segment (start 129.804 56.927) (end 131.054 58.177) (width 0.5) (layer "F.Cu") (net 2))
 (segment (start 142.405 83.523) (end 139.3952 83.523) (width 0.5) (layer "F.Cu") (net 2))
 (segment (start 155.651 65.8488) (end 155.651 57.8488) (width 0.5) (layer "F.Cu") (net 2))
 (segment (start 127.9435 93.726) (end 126.7244 92.5069) (width 0.5) (layer "F.Cu") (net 2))
 (segment (start 155.651 89.429) (end 154.08 91) (width 0.5) (layer "F.Cu") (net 2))
 (segment (start 154.9192 95.3008) (end 158.1912 92.0288) (width 0.5) (layer "F.Cu") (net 2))
 (segment (start 134.8412 41.1988) (end 132.54 43.5) (width 0.5) (layer "F.Cu") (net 2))
 (segment (start 131.054 58.177) (end 131.054 68.377) (width 0.5) (layer "F.Cu") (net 2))
 (segment (start 137.008 83.5152) (end 135.716 83.5152) (width 0.5) (layer "F.Cu") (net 2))
 (segment (start 129.804 51.847) (end 129.804 54.387) (width 0.5) (layer "F.Cu") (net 2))
 (segment (start 158.1912 92.0288) (end 158.1912 89.429) (width 0.5) (layer "F.Cu") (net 2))
 (segment (start 158.5 63) (end 165 63) (width 0.5) (layer "F.Cu") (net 2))
 (segment (start 152.1966 41.1988) (end 134.8412 41.1988) (width 0.5) (layer "F.Cu") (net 2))
 (segment (start 129.5183 95.3008) (end 154.9192 95.3008) (width 0.5) (layer "F.Cu") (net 2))
 (segment (start 142.0368 53.6828) (end 142.0368 56.6928) (width 0.5) (layer "F.Cu") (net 2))
 (segment (start 155.651 65.8488) (end 155.651 89.429) (width 0.5) (layer "F.Cu") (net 2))
 (segment (start 139.3952 83.523) (end 137.015 83.523) (width 0.5) (layer "F.Cu") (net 2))
 (segment (start 155.651 57.8488) (end 158.5 55) (width 0.5) (layer "F.Cu") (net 2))
 (segment (start 142.0368 53.6828) (end 142.0368 70.6628) (width 0.5) (layer "F.Cu") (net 2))
 (segment (start 155.651 57.8488) (end 155.651 44.6532) (width 0.5) (layer "F.Cu") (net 2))
 (segment (start 155.651 44.6532) (end 152.1966 41.1988) (width 0.5) (layer "F.Cu") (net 2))
 (segment (start 158.1912 89.429) (end 155.651 89.429) (width 0.5) (layer "F.Cu") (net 2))
 (segment (start 127.9435 93.726) (end 129.5183 95.3008) (width 0.5) (layer "F.Cu") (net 2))
 (via (at 131.007 78.3319) (size 0.8) (drill 0.4) (layers "F.Cu" "B.Cu") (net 2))
 (segment (start 131.007 79.264) (end 131.007 78.3319) (width 0.5) (layer "B.Cu") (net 2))
 (segment (start 129.804 77.1289) (end 129.804 69.627) (width 0.5) (layer "B.Cu") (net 2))
 (segment (start 131.007 78.3319) (end 129.804 77.1289) (width 0.5) (layer "B.Cu") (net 2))
 (segment (start 132.0292 48.0568) (end 128.1684 44.196) (width 0.5) (layer "B.Cu") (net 12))
 (segment (start 131.007 80.534) (end 131.634 80.534) (width 0.5) (layer "B.Cu") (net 12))
 (segment (start 132.442 59.3788) (end 137.424 54.3968) (width 0.5) (layer "B.Cu") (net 12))
 (segment (start 124.9725 85.9388) (end 124.9725 94.0676) (width 0.5) (layer "B.Cu") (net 12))
 (segment (start 131.634 80.534) (end 132.442 79.7258) (width 0.5) (layer "B.Cu") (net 12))
 (segment (start 129.0828 41.8084) (end 135.9284 41.8084) (width 0.5) (layer "B.Cu") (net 12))
 (segment (start 141.376 56.4896) (end 142.8496 56.4896) (width 0.5) (layer "B.Cu") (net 12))
 (segment (start 135.9284 41.8084) (end 137.62 43.5) (width 0.5) (layer "B.Cu") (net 12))
 (segment (start 144.374 54.8636) (end 144.374 48.6664) (width 0.5) (layer "B.Cu") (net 12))
 (segment (start 145.9996 56.4896) (end 146 56.4896) (width 0.5) (layer "B.Cu") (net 12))
 (segment (start 124.9725 94.0676) (end 125.1707 94.2658) (width 0.5) (layer "B.Cu") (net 12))
 (segment (start 128.1684 44.196) (end 128.1684 42.7228) (width 0.5) (layer "B.Cu") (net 12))
 (segment (start 137.424 54.387) (end 139.274 54.387) (width 0.5) (layer "B.Cu") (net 12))
 (segment (start 125.1707 94.2658) (end 145.7342 94.2658) (width 0.5) (layer "B.Cu") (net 12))
 (segment (start 146 56.4896) (end 144.374 54.8636) (width 0.5) (layer "B.Cu") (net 12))
 (segment (start 132.442 79.7258) (end 132.442 59.3788) (width 0.5) (layer "B.Cu") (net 12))
 (segment (start 128.1684 42.7228) (end 129.0828 41.8084) (width 0.5) (layer "B.Cu") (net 12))
 (segment (start 131.007 80.534) (end 130.3773 80.534) (width 0.5) (layer "B.Cu") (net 12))
 (segment (start 130.3773 80.534) (end 124.9725 85.9388) (width 0.5) (layer "B.Cu") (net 12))
 (segment (start 145.7342 94.2658) (end 149 91) (width 0.5) (layer "B.Cu") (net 12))
 (segment (start 142.8496 56.4896) (end 145.9996 56.4896) (width 0.5) (layer "B.Cu") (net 12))
 (segment (start 139.274 54.387) (end 141.376 56.4896) (width 0.5) (layer "B.Cu") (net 12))
 (segment (start 144.374 48.6664) (end 143.7644 48.0568) (width 0.5) (layer "B.Cu") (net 12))
 (segment (start 143.7644 48.0568) (end 132.0292 48.0568) (width 0.5) (layer "B.Cu") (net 12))
 (segment (start 137.424 54.3968) (end 137.424 54.387) (width 0.5) (layer "B.Cu") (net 12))
 (segment (start 135.32 80.534) (end 134.512 79.7258) (width 0.5) (layer "B.Cu") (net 13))
 (segment (start 147.726 54.5592) (end 149.606 56.4388) (width 0.5) (layer "B.Cu") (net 13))
 (segment (start 141.1732 80.6332) (end 151.54 91) (width 0.5) (layer "B.Cu") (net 13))
 (segment (start 145.238346 46.482) (end 147.726 48.969654) (width 0.5) (layer "B.Cu") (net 13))
 (segment (start 138.062 46.482) (end 145.238346 46.482) (width 0.5) (layer "B.Cu") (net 13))
 (segment (start 140.036 56.927) (end 141.072 57.9628) (width 0.5) (layer "B.Cu") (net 13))
 (segment (start 135.947 80.534) (end 135.32 80.534) (width 0.5) (layer "B.Cu") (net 13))
 (segment (start 134.512 59.839) (end 137.424 56.927) (width 0.5) (layer "B.Cu") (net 13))
 (segment (start 147.726 48.969654) (end 147.726 54.5592) (width 0.5) (layer "B.Cu") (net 13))
 (segment (start 134.512 79.7258) (end 134.512 59.839) (width 0.5) (layer "B.Cu") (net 13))
 (segment (start 135.947 80.534) (end 141.0876 80.534) (width 0.5) (layer "B.Cu") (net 13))
 (segment (start 148.082 57.9628) (end 149.606 56.4388) (width 0.5) (layer "B.Cu") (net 13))
 (segment (start 141.072 57.9628) (end 148.082 57.9628) (width 0.5) (layer "B.Cu") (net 13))
 (segment (start 135.08 43.5) (end 138.062 46.482) (width 0.5) (layer "B.Cu") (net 13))
 (segment (start 141.1732 80.6196) (end 141.1732 80.6332) (width 0.5) (layer "B.Cu") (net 13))
 (segment (start 137.424 56.927) (end 140.036 56.927) (width 0.5) (layer "B.Cu") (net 13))
 (segment (start 141.0876 80.534) (end 141.1732 80.6196) (width 0.5) (layer "B.Cu") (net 13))
 (segment (start 137.424 62.007) (end 139.964 62.007) (width 0.5) (layer "B.Cu") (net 4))
 (segment (start 156.817 65.817) (end 158.5 67.5) (width 0.5) (layer "B.Cu") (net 5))
 (segment (start 146.4181 63.1729) (end 146.4181 65.0286) (width 0.5) (layer "B.Cu") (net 5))
 (segment (start 147.584 62.007) (end 146.4181 63.1729) (width 0.5) (layer "B.Cu") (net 5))
 (segment (start 158.5 67.5) (end 165 67.5) (width 0.5) (layer "B.Cu") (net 5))
 (segment (start 146.4181 65.0286) (end 147.2065 65.817) (width 0.5) (layer "B.Cu") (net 5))
 (segment (start 147.2065 65.817) (end 156.817 65.817) (width 0.5) (layer "B.Cu") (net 5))
 (segment (start 137.424 64.547) (end 139.964 64.547) (width 0.5) (layer "B.Cu") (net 17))
 (segment (start 147.584 63.6831) (end 158.5 52.7671) (width 0.5) (layer "B.Cu") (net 1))
 (segment (start 147.584 64.547) (end 147.584 63.6831) (width 0.5) (layer "B.Cu") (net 1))
 (segment (start 158.5 52.7671) (end 158.5 50.5) (width 0.5) (layer "B.Cu") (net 1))
 (segment (start 158.5 50.5) (end 165 50.5) (width 0.5) (layer "B.Cu") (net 1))
 (segment (start 137.424 67.087) (end 139.964 67.087) (width 0.5) (layer "B.Cu") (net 16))
 (segment (start 137.424 69.627) (end 139.964 69.627) (width 0.5) (layer "B.Cu") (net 8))
 (segment (start 129.804 67.087) (end 127.264 67.087) (width 0.5) (layer "B.Cu") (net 10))
 (segment (start 129.804 64.547) (end 127.264 64.547) (width 0.5) (layer "B.Cu") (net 6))
 (segment (start 129.804 62.007) (end 127.264 62.007) (width 0.5) (layer "B.Cu") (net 15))
 (segment (start 129.804 59.467) (end 127.264 59.467) (width 0.5) (layer "B.Cu") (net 14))
 (segment (start 133.858 86.9188) (end 135.534 88.5952) (width 0.5) (layer "B.Cu") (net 23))
 (segment (start 133.858 83.062) (end 133.858 86.9188) (width 0.5) (layer "B.Cu") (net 23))
 (segment (start 135.534 88.5952) (end 137.813 88.5952) (width 0.5) (layer "B.Cu") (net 23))
 (segment (start 141.7244 92.5068) (end 141.724 92.5068) (width 0.5) (layer "B.Cu") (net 23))
 (segment (start 135.116 81.804) (end 133.858 83.062) (width 0.5) (layer "B.Cu") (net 23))
 (segment (start 137.813 88.5952) (end 141.724 92.5068) (width 0.5) (layer "B.Cu") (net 23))
 (segment (start 135.947 81.804) (end 135.116 81.804) (width 0.5) (layer "B.Cu") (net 23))
 (segment (start 136.7244 92.5068) (end 136.724 92.5068) (width 0.5) (layer "B.Cu") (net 22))
 (segment (start 136.724 92.5068) (end 132.791 88.5736) (width 0.5) (layer "B.Cu") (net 22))
 (segment (start 132.791 82.9614) (end 131.634 81.804) (width 0.5) (layer "B.Cu") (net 22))
 (segment (start 132.791 88.5736) (end 132.791 82.9614) (width 0.5) (layer "B.Cu") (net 22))
 (segment (start 131.634 81.804) (end 131.007 81.804) (width 0.5) (layer "B.Cu") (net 22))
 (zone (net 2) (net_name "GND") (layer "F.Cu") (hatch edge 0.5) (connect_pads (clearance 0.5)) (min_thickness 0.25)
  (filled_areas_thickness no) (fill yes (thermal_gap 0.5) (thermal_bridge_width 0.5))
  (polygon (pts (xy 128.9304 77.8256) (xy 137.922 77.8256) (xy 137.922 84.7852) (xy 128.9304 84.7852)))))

